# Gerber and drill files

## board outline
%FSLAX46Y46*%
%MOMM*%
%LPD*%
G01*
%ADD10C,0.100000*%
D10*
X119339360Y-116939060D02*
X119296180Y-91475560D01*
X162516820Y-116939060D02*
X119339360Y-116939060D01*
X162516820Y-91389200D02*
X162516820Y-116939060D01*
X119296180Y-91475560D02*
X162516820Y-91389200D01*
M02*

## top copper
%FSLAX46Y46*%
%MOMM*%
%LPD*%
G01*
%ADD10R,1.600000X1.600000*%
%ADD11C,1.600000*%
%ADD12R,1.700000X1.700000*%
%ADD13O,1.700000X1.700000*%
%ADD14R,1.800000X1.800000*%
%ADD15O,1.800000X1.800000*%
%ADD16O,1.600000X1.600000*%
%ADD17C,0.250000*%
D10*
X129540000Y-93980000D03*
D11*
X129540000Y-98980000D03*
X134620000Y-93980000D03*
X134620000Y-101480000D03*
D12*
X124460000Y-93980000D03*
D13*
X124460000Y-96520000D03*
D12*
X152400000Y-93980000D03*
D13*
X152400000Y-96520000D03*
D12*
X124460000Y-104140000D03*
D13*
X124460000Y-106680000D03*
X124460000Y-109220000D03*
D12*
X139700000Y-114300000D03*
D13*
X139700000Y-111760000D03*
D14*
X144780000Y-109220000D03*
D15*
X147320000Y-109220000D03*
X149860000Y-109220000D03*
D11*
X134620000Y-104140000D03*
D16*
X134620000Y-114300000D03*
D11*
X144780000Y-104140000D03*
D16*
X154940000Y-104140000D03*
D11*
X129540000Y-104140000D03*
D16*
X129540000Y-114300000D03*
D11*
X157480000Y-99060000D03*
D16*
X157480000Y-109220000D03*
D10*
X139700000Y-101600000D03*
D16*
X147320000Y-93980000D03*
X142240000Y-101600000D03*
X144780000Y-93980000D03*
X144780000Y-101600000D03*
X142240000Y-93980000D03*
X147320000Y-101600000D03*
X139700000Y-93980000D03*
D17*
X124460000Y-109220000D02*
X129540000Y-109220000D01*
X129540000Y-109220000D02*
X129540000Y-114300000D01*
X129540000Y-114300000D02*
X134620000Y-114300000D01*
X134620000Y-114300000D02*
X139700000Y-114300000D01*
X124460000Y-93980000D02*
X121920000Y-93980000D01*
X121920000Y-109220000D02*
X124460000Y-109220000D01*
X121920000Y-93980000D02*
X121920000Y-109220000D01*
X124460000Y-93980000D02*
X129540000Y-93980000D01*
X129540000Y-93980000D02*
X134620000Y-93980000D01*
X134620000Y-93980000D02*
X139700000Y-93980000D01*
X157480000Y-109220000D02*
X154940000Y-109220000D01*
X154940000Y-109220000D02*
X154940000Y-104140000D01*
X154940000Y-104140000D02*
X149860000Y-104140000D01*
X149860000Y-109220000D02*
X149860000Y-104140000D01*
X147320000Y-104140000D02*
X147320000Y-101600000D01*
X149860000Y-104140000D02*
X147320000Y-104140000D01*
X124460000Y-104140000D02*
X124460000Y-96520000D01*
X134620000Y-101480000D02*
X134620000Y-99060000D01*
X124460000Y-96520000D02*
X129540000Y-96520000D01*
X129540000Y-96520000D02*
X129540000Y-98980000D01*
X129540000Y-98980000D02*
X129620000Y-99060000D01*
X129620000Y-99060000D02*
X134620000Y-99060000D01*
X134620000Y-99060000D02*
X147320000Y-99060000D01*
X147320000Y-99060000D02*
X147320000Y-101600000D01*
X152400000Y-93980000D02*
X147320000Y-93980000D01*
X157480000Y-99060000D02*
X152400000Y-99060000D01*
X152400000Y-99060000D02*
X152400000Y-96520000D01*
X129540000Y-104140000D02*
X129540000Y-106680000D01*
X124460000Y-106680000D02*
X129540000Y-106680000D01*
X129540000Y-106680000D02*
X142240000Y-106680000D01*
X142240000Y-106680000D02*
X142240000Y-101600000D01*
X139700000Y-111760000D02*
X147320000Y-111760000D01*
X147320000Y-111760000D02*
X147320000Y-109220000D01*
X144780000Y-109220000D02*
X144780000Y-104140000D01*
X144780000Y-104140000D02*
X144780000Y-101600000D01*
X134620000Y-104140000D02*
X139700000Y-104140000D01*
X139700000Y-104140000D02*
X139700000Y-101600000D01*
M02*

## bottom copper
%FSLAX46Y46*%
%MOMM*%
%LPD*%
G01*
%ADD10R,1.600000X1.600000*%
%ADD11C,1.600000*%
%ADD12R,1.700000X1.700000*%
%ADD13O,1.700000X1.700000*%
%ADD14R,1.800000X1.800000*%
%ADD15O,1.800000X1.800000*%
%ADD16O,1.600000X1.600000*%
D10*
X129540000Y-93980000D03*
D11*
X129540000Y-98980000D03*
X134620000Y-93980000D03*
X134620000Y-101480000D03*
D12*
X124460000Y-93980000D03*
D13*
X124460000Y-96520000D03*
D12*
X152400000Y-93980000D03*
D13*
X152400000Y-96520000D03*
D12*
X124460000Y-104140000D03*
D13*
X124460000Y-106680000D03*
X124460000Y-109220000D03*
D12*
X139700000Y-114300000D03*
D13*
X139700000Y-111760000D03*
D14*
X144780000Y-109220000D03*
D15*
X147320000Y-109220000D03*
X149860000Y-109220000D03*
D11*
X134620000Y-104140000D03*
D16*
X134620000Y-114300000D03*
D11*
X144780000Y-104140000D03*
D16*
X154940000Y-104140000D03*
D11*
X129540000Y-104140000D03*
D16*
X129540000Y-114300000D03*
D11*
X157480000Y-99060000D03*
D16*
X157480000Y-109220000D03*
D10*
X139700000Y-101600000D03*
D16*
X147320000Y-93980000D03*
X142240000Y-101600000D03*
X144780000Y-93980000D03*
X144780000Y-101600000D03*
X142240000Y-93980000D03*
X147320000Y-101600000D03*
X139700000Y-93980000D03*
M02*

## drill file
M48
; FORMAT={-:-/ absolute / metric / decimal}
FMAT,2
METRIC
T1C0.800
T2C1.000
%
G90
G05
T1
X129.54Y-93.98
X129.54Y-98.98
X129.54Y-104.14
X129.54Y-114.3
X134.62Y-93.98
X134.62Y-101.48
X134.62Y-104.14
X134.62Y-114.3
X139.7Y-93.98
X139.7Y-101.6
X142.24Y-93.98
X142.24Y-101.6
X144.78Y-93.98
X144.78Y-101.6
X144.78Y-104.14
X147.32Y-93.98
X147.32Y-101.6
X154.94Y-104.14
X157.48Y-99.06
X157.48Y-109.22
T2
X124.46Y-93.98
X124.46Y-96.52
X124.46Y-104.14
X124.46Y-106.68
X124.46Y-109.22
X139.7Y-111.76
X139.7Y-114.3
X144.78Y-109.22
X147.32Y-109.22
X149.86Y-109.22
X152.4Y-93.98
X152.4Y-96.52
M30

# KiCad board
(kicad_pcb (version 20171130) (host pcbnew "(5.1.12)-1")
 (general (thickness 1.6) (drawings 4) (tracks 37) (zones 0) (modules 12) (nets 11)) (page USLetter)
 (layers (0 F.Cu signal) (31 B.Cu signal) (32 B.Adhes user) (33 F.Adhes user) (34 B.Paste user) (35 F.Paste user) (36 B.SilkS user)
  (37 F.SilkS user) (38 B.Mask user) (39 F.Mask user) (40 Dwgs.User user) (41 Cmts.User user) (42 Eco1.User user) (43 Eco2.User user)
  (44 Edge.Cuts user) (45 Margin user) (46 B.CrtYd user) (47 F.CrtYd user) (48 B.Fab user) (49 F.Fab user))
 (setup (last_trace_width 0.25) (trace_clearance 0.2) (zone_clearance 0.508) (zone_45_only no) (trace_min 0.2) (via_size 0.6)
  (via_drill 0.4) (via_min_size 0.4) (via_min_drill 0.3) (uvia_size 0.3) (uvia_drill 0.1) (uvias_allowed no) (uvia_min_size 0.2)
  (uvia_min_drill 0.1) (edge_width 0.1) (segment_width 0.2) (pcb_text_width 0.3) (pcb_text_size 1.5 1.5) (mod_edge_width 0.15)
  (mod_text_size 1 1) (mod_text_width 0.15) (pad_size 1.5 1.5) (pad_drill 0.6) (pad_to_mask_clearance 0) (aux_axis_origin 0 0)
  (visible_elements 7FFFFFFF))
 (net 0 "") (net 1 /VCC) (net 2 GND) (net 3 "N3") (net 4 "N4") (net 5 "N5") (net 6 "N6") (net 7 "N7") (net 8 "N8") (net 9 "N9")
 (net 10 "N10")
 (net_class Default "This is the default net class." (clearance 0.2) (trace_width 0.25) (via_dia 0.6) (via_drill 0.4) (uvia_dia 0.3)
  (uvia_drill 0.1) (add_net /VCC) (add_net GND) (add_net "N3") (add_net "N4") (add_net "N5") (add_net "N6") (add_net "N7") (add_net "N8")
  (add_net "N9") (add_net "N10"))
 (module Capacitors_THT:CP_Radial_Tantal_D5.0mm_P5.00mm (layer F.Cu) (at 129.54 93.98 270)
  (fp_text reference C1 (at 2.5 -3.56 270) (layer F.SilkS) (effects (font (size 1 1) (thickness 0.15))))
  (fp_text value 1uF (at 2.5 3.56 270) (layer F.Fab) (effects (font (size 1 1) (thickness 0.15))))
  (pad 1 thru_hole rect (at 0 0 270) (size 1.6 1.6) (drill 0.8) (layers *.Cu *.Mask) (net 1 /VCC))
  (pad 2 thru_hole circle (at 5 0 270) (size 1.6 1.6) (drill 0.8) (layers *.Cu *.Mask) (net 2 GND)))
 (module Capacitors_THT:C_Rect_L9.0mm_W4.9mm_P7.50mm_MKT (layer F.Cu) (at 134.62 93.98 270)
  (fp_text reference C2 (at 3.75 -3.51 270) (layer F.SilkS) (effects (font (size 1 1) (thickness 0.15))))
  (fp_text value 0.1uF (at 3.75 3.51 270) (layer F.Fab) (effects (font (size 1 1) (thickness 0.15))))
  (pad 1 thru_hole circle (at 0 0 270) (size 1.6 1.6) (drill 0.8) (layers *.Cu *.Mask) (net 1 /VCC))
  (pad 2 thru_hole circle (at 7.5 0 270) (size 1.6 1.6) (drill 0.8) (layers *.Cu *.Mask) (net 2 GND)))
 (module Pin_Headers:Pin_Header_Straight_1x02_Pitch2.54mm (layer F.Cu) (at 124.46 93.98)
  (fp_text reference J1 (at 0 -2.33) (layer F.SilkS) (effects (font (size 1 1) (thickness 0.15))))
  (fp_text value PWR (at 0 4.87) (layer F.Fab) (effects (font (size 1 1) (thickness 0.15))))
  (pad 1 thru_hole rect (at 0 0) (size 1.7 1.7) (drill 1) (layers *.Cu *.Mask) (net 1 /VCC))
  (pad 2 thru_hole oval (at 0 2.54) (size 1.7 1.7) (drill 1) (layers *.Cu *.Mask) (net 2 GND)))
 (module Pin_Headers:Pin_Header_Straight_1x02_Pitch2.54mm (layer F.Cu) (at 152.4 93.98)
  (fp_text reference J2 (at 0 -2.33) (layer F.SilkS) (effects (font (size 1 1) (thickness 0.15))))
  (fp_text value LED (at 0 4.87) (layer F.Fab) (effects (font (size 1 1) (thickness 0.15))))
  (pad 1 thru_hole rect (at 0 0) (size 1.7 1.7) (drill 1) (layers *.Cu *.Mask) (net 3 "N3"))
  (pad 2 thru_hole oval (at 0 2.54) (size 1.7 1.7) (drill 1) (layers *.Cu *.Mask) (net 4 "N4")))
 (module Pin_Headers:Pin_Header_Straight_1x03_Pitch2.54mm (layer F.Cu) (at 124.46 104.14)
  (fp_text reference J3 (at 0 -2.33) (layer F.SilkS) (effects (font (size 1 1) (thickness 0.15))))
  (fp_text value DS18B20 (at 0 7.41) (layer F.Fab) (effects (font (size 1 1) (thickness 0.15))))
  (pad 1 thru_hole rect (at 0 0) (size 1.7 1.7) (drill 1) (layers *.Cu *.Mask) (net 2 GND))
  (pad 2 thru_hole oval (at 0 2.54) (size 1.7 1.7) (drill 1) (layers *.Cu *.Mask) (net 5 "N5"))
  (pad 3 thru_hole oval (at 0 5.08) (size 1.7 1.7) (drill 1) (layers *.Cu *.Mask) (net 1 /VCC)))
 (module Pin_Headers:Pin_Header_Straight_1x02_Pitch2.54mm (layer F.Cu) (at 139.7 114.3 180)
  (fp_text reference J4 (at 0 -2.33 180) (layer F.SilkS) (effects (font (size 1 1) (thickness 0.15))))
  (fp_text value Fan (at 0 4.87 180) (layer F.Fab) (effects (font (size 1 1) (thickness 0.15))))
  (pad 1 thru_hole rect (at 0 0 180) (size 1.7 1.7) (drill 1) (layers *.Cu *.Mask) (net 1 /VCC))
  (pad 2 thru_hole oval (at 0 2.54 180) (size 1.7 1.7) (drill 1) (layers *.Cu *.Mask) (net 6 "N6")))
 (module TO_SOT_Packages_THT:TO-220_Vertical (layer F.Cu) (at 144.78 109.22)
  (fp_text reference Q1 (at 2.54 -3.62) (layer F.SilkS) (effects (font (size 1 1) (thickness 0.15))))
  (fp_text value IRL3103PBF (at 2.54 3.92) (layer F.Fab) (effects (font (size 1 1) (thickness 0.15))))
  (pad 1 thru_hole rect (at 0 0) (size 1.8 1.8) (drill 1) (layers *.Cu *.Mask) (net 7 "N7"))
  (pad 2 thru_hole oval (at 2.54 0) (size 1.8 1.8) (drill 1) (layers *.Cu *.Mask) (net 6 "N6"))
  (pad 3 thru_hole oval (at 5.08 0) (size 1.8 1.8) (drill 1) (layers *.Cu *.Mask) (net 2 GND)))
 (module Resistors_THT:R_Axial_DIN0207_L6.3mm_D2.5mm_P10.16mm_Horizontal (layer F.Cu) (at 134.62 104.14 270)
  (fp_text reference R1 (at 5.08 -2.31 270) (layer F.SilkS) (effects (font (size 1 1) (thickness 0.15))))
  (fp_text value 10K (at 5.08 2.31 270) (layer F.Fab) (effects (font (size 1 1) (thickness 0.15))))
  (pad 1 thru_hole circle (at 0 0 270) (size 1.6 1.6) (drill 0.8) (layers *.Cu *.Mask) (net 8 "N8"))
  (pad 2 thru_hole oval (at 10.16 0 270) (size 1.6 1.6) (drill 0.8) (layers *.Cu *.Mask) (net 1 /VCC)))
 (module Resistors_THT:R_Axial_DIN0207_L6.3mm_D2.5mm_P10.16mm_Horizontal (layer F.Cu) (at 144.78 104.14)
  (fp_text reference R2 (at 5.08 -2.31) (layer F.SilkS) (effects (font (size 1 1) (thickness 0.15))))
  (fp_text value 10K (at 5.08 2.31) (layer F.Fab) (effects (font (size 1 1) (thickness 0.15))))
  (pad 1 thru_hole circle (at 0 0) (size 1.6 1.6) (drill 0.8) (layers *.Cu *.Mask) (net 7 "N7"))
  (pad 2 thru_hole oval (at 10.16 0) (size 1.6 1.6) (drill 0.8) (layers *.Cu *.Mask) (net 2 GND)))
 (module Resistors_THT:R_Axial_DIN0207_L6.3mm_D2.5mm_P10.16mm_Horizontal (layer F.Cu) (at 129.54 104.14 270)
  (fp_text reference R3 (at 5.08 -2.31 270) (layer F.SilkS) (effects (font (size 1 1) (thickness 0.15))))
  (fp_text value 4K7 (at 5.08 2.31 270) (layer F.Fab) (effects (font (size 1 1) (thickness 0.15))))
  (pad 1 thru_hole circle (at 0 0 270) (size 1.6 1.6) (drill 0.8) (layers *.Cu *.Mask) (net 5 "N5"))
  (pad 2 thru_hole oval (at 10.16 0 270) (size 1.6 1.6) (drill 0.8) (layers *.Cu *.Mask) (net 1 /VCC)))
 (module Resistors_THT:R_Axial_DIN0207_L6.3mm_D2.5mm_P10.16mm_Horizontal (layer F.Cu) (at 157.48 99.06 270)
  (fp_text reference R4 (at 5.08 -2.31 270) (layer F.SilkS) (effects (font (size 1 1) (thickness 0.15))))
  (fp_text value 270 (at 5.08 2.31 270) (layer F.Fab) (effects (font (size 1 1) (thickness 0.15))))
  (pad 1 thru_hole circle (at 0 0 270) (size 1.6 1.6) (drill 0.8) (layers *.Cu *.Mask) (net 4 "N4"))
  (pad 2 thru_hole oval (at 10.16 0 270) (size 1.6 1.6) (drill 0.8) (layers *.Cu *.Mask) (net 2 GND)))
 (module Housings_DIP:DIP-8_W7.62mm (layer F.Cu) (at 139.7 101.6 90)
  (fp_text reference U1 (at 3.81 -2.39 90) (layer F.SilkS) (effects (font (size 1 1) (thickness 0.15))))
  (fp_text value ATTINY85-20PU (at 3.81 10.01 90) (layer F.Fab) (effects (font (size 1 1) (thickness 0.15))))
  (pad 1 thru_hole rect (at 0 0 90) (size 1.6 1.6) (drill 0.8) (layers *.Cu *.Mask) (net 8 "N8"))
  (pad 5 thru_hole oval (at 7.62 7.62 90) (size 1.6 1.6) (drill 0.8) (layers *.Cu *.Mask) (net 3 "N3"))
  (pad 2 thru_hole oval (at 0 2.54 90) (size 1.6 1.6) (drill 0.8) (layers *.Cu *.Mask) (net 5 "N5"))
  (pad 6 thru_hole oval (at 7.62 5.08 90) (size 1.6 1.6) (drill 0.8) (layers *.Cu *.Mask) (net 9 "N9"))
  (pad 3 thru_hole oval (at 0 5.08 90) (size 1.6 1.6) (drill 0.8) (layers *.Cu *.Mask) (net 7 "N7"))
  (pad 7 thru_hole oval (at 7.62 2.54 90) (size 1.6 1.6) (drill 0.8) (layers *.Cu *.Mask) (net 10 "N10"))
  (pad 4 thru_hole oval (at 0 7.62 90) (size 1.6 1.6) (drill 0.8) (layers *.Cu *.Mask) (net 2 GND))
  (pad 8 thru_hole oval (at 7.62 0 90) (size 1.6 1.6) (drill 0.8) (layers *.Cu *.Mask) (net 1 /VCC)))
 (gr_line (start 119.33936 116.93906) (end 119.29618 91.47556) (layer Edge.Cuts) (width 0.1))
 (gr_line (start 162.51682 116.93906) (end 119.33936 116.93906) (layer Edge.Cuts) (width 0.1))
 (gr_line (start 162.51682 91.3892) (end 162.51682 116.93906) (layer Edge.Cuts) (width 0.1))
 (gr_line (start 119.29618 91.47556) (end 162.51682 91.3892) (layer Edge.Cuts) (width 0.1))
 (segment (start 124.46 109.22) (end 129.54 109.22) (width 0.25) (layer F.Cu) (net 1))
 (segment (start 129.54 109.22) (end 129.54 114.3) (width 0.25) (layer F.Cu) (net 1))
 (segment (start 129.54 114.3) (end 134.62 114.3) (width 0.25) (layer F.Cu) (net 1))
 (segment (start 134.62 114.3) (end 139.7 114.3) (width 0.25) (layer F.Cu) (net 1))
 (segment (start 124.46 93.98) (end 121.92 93.98) (width 0.25) (layer F.Cu) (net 1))
 (segment (start 121.92 109.22) (end 124.46 109.22) (width 0.25) (layer F.Cu) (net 1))
 (segment (start 121.92 93.98) (end 121.92 109.22) (width 0.25) (layer F.Cu) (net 1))
 (segment (start 124.46 93.98) (end 129.54 93.98) (width 0.25) (layer F.Cu) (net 1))
 (segment (start 129.54 93.98) (end 134.62 93.98) (width 0.25) (layer F.Cu) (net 1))
 (segment (start 134.62 93.98) (end 139.7 93.98) (width 0.25) (layer F.Cu) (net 1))
 (segment (start 157.48 109.22) (end 154.94 109.22) (width 0.25) (layer F.Cu) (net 2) (status 400000))
 (segment (start 154.94 109.22) (end 154.94 104.14) (width 0.25) (layer F.Cu) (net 2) (status 800000))
 (segment (start 154.94 104.14) (end 149.86 104.14) (width 0.25) (layer F.Cu) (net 2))
 (segment (start 149.86 109.22) (end 149.86 104.14) (width 0.25) (layer F.Cu) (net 2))
 (segment (start 147.32 104.14) (end 147.32 101.6) (width 0.25) (layer F.Cu) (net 2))
 (segment (start 149.86 104.14) (end 147.32 104.14) (width 0.25) (layer F.Cu) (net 2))
 (segment (start 124.46 104.14) (end 124.46 96.52) (width 0.25) (layer F.Cu) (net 2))
 (segment (start 134.62 101.48) (end 134.62 99.06) (width 0.25) (layer F.Cu) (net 2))
 (segment (start 124.46 96.52) (end 129.54 96.52) (width 0.25) (layer F.Cu) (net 2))
 (segment (start 129.54 96.52) (end 129.54 98.98) (width 0.25) (layer F.Cu) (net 2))
 (segment (start 129.54 98.98) (end 129.62 99.06) (width 0.25) (layer F.Cu) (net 2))
 (segment (start 129.62 99.06) (end 134.62 99.06) (width 0.25) (layer F.Cu) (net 2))
 (segment (start 134.62 99.06) (end 147.32 99.06) (width 0.25) (layer F.Cu) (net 2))
 (segment (start 147.32 99.06) (end 147.32 101.6) (width 0.25) (layer F.Cu) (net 2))
 (segment (start 152.4 93.98) (end 147.32 93.98) (width 0.25) (layer F.Cu) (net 3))
 (segment (start 157.48 99.06) (end 152.4 99.06) (width 0.25) (layer F.Cu) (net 4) (status 400000))
 (segment (start 152.4 99.06) (end 152.4 96.52) (width 0.25) (layer F.Cu) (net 4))
 (segment (start 129.54 104.14) (end 129.54 106.68) (width 0.25) (layer F.Cu) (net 5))
 (segment (start 124.46 106.68) (end 129.54 106.68) (width 0.25) (layer F.Cu) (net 5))
 (segment (start 129.54 106.68) (end 142.24 106.68) (width 0.25) (layer F.Cu) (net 5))
 (segment (start 142.24 106.68) (end 142.24 101.6) (width 0.25) (layer F.Cu) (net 5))
 (segment (start 139.7 111.76) (end 147.32 111.76) (width 0.25) (layer F.Cu) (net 6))
 (segment (start 147.32 111.76) (end 147.32 109.22) (width 0.25) (layer F.Cu) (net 6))
 (segment (start 144.78 109.22) (end 144.78 104.14) (width 0.25) (layer F.Cu) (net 7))
 (segment (start 144.78 104.14) (end 144.78 101.6) (width 0.25) (layer F.Cu) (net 7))
 (segment (start 134.62 104.14) (end 139.7 104.14) (width 0.25) (layer F.Cu) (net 8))
 (segment (start 139.7 104.14) (end 139.7 101.6) (width 0.25) (layer F.Cu) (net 8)))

